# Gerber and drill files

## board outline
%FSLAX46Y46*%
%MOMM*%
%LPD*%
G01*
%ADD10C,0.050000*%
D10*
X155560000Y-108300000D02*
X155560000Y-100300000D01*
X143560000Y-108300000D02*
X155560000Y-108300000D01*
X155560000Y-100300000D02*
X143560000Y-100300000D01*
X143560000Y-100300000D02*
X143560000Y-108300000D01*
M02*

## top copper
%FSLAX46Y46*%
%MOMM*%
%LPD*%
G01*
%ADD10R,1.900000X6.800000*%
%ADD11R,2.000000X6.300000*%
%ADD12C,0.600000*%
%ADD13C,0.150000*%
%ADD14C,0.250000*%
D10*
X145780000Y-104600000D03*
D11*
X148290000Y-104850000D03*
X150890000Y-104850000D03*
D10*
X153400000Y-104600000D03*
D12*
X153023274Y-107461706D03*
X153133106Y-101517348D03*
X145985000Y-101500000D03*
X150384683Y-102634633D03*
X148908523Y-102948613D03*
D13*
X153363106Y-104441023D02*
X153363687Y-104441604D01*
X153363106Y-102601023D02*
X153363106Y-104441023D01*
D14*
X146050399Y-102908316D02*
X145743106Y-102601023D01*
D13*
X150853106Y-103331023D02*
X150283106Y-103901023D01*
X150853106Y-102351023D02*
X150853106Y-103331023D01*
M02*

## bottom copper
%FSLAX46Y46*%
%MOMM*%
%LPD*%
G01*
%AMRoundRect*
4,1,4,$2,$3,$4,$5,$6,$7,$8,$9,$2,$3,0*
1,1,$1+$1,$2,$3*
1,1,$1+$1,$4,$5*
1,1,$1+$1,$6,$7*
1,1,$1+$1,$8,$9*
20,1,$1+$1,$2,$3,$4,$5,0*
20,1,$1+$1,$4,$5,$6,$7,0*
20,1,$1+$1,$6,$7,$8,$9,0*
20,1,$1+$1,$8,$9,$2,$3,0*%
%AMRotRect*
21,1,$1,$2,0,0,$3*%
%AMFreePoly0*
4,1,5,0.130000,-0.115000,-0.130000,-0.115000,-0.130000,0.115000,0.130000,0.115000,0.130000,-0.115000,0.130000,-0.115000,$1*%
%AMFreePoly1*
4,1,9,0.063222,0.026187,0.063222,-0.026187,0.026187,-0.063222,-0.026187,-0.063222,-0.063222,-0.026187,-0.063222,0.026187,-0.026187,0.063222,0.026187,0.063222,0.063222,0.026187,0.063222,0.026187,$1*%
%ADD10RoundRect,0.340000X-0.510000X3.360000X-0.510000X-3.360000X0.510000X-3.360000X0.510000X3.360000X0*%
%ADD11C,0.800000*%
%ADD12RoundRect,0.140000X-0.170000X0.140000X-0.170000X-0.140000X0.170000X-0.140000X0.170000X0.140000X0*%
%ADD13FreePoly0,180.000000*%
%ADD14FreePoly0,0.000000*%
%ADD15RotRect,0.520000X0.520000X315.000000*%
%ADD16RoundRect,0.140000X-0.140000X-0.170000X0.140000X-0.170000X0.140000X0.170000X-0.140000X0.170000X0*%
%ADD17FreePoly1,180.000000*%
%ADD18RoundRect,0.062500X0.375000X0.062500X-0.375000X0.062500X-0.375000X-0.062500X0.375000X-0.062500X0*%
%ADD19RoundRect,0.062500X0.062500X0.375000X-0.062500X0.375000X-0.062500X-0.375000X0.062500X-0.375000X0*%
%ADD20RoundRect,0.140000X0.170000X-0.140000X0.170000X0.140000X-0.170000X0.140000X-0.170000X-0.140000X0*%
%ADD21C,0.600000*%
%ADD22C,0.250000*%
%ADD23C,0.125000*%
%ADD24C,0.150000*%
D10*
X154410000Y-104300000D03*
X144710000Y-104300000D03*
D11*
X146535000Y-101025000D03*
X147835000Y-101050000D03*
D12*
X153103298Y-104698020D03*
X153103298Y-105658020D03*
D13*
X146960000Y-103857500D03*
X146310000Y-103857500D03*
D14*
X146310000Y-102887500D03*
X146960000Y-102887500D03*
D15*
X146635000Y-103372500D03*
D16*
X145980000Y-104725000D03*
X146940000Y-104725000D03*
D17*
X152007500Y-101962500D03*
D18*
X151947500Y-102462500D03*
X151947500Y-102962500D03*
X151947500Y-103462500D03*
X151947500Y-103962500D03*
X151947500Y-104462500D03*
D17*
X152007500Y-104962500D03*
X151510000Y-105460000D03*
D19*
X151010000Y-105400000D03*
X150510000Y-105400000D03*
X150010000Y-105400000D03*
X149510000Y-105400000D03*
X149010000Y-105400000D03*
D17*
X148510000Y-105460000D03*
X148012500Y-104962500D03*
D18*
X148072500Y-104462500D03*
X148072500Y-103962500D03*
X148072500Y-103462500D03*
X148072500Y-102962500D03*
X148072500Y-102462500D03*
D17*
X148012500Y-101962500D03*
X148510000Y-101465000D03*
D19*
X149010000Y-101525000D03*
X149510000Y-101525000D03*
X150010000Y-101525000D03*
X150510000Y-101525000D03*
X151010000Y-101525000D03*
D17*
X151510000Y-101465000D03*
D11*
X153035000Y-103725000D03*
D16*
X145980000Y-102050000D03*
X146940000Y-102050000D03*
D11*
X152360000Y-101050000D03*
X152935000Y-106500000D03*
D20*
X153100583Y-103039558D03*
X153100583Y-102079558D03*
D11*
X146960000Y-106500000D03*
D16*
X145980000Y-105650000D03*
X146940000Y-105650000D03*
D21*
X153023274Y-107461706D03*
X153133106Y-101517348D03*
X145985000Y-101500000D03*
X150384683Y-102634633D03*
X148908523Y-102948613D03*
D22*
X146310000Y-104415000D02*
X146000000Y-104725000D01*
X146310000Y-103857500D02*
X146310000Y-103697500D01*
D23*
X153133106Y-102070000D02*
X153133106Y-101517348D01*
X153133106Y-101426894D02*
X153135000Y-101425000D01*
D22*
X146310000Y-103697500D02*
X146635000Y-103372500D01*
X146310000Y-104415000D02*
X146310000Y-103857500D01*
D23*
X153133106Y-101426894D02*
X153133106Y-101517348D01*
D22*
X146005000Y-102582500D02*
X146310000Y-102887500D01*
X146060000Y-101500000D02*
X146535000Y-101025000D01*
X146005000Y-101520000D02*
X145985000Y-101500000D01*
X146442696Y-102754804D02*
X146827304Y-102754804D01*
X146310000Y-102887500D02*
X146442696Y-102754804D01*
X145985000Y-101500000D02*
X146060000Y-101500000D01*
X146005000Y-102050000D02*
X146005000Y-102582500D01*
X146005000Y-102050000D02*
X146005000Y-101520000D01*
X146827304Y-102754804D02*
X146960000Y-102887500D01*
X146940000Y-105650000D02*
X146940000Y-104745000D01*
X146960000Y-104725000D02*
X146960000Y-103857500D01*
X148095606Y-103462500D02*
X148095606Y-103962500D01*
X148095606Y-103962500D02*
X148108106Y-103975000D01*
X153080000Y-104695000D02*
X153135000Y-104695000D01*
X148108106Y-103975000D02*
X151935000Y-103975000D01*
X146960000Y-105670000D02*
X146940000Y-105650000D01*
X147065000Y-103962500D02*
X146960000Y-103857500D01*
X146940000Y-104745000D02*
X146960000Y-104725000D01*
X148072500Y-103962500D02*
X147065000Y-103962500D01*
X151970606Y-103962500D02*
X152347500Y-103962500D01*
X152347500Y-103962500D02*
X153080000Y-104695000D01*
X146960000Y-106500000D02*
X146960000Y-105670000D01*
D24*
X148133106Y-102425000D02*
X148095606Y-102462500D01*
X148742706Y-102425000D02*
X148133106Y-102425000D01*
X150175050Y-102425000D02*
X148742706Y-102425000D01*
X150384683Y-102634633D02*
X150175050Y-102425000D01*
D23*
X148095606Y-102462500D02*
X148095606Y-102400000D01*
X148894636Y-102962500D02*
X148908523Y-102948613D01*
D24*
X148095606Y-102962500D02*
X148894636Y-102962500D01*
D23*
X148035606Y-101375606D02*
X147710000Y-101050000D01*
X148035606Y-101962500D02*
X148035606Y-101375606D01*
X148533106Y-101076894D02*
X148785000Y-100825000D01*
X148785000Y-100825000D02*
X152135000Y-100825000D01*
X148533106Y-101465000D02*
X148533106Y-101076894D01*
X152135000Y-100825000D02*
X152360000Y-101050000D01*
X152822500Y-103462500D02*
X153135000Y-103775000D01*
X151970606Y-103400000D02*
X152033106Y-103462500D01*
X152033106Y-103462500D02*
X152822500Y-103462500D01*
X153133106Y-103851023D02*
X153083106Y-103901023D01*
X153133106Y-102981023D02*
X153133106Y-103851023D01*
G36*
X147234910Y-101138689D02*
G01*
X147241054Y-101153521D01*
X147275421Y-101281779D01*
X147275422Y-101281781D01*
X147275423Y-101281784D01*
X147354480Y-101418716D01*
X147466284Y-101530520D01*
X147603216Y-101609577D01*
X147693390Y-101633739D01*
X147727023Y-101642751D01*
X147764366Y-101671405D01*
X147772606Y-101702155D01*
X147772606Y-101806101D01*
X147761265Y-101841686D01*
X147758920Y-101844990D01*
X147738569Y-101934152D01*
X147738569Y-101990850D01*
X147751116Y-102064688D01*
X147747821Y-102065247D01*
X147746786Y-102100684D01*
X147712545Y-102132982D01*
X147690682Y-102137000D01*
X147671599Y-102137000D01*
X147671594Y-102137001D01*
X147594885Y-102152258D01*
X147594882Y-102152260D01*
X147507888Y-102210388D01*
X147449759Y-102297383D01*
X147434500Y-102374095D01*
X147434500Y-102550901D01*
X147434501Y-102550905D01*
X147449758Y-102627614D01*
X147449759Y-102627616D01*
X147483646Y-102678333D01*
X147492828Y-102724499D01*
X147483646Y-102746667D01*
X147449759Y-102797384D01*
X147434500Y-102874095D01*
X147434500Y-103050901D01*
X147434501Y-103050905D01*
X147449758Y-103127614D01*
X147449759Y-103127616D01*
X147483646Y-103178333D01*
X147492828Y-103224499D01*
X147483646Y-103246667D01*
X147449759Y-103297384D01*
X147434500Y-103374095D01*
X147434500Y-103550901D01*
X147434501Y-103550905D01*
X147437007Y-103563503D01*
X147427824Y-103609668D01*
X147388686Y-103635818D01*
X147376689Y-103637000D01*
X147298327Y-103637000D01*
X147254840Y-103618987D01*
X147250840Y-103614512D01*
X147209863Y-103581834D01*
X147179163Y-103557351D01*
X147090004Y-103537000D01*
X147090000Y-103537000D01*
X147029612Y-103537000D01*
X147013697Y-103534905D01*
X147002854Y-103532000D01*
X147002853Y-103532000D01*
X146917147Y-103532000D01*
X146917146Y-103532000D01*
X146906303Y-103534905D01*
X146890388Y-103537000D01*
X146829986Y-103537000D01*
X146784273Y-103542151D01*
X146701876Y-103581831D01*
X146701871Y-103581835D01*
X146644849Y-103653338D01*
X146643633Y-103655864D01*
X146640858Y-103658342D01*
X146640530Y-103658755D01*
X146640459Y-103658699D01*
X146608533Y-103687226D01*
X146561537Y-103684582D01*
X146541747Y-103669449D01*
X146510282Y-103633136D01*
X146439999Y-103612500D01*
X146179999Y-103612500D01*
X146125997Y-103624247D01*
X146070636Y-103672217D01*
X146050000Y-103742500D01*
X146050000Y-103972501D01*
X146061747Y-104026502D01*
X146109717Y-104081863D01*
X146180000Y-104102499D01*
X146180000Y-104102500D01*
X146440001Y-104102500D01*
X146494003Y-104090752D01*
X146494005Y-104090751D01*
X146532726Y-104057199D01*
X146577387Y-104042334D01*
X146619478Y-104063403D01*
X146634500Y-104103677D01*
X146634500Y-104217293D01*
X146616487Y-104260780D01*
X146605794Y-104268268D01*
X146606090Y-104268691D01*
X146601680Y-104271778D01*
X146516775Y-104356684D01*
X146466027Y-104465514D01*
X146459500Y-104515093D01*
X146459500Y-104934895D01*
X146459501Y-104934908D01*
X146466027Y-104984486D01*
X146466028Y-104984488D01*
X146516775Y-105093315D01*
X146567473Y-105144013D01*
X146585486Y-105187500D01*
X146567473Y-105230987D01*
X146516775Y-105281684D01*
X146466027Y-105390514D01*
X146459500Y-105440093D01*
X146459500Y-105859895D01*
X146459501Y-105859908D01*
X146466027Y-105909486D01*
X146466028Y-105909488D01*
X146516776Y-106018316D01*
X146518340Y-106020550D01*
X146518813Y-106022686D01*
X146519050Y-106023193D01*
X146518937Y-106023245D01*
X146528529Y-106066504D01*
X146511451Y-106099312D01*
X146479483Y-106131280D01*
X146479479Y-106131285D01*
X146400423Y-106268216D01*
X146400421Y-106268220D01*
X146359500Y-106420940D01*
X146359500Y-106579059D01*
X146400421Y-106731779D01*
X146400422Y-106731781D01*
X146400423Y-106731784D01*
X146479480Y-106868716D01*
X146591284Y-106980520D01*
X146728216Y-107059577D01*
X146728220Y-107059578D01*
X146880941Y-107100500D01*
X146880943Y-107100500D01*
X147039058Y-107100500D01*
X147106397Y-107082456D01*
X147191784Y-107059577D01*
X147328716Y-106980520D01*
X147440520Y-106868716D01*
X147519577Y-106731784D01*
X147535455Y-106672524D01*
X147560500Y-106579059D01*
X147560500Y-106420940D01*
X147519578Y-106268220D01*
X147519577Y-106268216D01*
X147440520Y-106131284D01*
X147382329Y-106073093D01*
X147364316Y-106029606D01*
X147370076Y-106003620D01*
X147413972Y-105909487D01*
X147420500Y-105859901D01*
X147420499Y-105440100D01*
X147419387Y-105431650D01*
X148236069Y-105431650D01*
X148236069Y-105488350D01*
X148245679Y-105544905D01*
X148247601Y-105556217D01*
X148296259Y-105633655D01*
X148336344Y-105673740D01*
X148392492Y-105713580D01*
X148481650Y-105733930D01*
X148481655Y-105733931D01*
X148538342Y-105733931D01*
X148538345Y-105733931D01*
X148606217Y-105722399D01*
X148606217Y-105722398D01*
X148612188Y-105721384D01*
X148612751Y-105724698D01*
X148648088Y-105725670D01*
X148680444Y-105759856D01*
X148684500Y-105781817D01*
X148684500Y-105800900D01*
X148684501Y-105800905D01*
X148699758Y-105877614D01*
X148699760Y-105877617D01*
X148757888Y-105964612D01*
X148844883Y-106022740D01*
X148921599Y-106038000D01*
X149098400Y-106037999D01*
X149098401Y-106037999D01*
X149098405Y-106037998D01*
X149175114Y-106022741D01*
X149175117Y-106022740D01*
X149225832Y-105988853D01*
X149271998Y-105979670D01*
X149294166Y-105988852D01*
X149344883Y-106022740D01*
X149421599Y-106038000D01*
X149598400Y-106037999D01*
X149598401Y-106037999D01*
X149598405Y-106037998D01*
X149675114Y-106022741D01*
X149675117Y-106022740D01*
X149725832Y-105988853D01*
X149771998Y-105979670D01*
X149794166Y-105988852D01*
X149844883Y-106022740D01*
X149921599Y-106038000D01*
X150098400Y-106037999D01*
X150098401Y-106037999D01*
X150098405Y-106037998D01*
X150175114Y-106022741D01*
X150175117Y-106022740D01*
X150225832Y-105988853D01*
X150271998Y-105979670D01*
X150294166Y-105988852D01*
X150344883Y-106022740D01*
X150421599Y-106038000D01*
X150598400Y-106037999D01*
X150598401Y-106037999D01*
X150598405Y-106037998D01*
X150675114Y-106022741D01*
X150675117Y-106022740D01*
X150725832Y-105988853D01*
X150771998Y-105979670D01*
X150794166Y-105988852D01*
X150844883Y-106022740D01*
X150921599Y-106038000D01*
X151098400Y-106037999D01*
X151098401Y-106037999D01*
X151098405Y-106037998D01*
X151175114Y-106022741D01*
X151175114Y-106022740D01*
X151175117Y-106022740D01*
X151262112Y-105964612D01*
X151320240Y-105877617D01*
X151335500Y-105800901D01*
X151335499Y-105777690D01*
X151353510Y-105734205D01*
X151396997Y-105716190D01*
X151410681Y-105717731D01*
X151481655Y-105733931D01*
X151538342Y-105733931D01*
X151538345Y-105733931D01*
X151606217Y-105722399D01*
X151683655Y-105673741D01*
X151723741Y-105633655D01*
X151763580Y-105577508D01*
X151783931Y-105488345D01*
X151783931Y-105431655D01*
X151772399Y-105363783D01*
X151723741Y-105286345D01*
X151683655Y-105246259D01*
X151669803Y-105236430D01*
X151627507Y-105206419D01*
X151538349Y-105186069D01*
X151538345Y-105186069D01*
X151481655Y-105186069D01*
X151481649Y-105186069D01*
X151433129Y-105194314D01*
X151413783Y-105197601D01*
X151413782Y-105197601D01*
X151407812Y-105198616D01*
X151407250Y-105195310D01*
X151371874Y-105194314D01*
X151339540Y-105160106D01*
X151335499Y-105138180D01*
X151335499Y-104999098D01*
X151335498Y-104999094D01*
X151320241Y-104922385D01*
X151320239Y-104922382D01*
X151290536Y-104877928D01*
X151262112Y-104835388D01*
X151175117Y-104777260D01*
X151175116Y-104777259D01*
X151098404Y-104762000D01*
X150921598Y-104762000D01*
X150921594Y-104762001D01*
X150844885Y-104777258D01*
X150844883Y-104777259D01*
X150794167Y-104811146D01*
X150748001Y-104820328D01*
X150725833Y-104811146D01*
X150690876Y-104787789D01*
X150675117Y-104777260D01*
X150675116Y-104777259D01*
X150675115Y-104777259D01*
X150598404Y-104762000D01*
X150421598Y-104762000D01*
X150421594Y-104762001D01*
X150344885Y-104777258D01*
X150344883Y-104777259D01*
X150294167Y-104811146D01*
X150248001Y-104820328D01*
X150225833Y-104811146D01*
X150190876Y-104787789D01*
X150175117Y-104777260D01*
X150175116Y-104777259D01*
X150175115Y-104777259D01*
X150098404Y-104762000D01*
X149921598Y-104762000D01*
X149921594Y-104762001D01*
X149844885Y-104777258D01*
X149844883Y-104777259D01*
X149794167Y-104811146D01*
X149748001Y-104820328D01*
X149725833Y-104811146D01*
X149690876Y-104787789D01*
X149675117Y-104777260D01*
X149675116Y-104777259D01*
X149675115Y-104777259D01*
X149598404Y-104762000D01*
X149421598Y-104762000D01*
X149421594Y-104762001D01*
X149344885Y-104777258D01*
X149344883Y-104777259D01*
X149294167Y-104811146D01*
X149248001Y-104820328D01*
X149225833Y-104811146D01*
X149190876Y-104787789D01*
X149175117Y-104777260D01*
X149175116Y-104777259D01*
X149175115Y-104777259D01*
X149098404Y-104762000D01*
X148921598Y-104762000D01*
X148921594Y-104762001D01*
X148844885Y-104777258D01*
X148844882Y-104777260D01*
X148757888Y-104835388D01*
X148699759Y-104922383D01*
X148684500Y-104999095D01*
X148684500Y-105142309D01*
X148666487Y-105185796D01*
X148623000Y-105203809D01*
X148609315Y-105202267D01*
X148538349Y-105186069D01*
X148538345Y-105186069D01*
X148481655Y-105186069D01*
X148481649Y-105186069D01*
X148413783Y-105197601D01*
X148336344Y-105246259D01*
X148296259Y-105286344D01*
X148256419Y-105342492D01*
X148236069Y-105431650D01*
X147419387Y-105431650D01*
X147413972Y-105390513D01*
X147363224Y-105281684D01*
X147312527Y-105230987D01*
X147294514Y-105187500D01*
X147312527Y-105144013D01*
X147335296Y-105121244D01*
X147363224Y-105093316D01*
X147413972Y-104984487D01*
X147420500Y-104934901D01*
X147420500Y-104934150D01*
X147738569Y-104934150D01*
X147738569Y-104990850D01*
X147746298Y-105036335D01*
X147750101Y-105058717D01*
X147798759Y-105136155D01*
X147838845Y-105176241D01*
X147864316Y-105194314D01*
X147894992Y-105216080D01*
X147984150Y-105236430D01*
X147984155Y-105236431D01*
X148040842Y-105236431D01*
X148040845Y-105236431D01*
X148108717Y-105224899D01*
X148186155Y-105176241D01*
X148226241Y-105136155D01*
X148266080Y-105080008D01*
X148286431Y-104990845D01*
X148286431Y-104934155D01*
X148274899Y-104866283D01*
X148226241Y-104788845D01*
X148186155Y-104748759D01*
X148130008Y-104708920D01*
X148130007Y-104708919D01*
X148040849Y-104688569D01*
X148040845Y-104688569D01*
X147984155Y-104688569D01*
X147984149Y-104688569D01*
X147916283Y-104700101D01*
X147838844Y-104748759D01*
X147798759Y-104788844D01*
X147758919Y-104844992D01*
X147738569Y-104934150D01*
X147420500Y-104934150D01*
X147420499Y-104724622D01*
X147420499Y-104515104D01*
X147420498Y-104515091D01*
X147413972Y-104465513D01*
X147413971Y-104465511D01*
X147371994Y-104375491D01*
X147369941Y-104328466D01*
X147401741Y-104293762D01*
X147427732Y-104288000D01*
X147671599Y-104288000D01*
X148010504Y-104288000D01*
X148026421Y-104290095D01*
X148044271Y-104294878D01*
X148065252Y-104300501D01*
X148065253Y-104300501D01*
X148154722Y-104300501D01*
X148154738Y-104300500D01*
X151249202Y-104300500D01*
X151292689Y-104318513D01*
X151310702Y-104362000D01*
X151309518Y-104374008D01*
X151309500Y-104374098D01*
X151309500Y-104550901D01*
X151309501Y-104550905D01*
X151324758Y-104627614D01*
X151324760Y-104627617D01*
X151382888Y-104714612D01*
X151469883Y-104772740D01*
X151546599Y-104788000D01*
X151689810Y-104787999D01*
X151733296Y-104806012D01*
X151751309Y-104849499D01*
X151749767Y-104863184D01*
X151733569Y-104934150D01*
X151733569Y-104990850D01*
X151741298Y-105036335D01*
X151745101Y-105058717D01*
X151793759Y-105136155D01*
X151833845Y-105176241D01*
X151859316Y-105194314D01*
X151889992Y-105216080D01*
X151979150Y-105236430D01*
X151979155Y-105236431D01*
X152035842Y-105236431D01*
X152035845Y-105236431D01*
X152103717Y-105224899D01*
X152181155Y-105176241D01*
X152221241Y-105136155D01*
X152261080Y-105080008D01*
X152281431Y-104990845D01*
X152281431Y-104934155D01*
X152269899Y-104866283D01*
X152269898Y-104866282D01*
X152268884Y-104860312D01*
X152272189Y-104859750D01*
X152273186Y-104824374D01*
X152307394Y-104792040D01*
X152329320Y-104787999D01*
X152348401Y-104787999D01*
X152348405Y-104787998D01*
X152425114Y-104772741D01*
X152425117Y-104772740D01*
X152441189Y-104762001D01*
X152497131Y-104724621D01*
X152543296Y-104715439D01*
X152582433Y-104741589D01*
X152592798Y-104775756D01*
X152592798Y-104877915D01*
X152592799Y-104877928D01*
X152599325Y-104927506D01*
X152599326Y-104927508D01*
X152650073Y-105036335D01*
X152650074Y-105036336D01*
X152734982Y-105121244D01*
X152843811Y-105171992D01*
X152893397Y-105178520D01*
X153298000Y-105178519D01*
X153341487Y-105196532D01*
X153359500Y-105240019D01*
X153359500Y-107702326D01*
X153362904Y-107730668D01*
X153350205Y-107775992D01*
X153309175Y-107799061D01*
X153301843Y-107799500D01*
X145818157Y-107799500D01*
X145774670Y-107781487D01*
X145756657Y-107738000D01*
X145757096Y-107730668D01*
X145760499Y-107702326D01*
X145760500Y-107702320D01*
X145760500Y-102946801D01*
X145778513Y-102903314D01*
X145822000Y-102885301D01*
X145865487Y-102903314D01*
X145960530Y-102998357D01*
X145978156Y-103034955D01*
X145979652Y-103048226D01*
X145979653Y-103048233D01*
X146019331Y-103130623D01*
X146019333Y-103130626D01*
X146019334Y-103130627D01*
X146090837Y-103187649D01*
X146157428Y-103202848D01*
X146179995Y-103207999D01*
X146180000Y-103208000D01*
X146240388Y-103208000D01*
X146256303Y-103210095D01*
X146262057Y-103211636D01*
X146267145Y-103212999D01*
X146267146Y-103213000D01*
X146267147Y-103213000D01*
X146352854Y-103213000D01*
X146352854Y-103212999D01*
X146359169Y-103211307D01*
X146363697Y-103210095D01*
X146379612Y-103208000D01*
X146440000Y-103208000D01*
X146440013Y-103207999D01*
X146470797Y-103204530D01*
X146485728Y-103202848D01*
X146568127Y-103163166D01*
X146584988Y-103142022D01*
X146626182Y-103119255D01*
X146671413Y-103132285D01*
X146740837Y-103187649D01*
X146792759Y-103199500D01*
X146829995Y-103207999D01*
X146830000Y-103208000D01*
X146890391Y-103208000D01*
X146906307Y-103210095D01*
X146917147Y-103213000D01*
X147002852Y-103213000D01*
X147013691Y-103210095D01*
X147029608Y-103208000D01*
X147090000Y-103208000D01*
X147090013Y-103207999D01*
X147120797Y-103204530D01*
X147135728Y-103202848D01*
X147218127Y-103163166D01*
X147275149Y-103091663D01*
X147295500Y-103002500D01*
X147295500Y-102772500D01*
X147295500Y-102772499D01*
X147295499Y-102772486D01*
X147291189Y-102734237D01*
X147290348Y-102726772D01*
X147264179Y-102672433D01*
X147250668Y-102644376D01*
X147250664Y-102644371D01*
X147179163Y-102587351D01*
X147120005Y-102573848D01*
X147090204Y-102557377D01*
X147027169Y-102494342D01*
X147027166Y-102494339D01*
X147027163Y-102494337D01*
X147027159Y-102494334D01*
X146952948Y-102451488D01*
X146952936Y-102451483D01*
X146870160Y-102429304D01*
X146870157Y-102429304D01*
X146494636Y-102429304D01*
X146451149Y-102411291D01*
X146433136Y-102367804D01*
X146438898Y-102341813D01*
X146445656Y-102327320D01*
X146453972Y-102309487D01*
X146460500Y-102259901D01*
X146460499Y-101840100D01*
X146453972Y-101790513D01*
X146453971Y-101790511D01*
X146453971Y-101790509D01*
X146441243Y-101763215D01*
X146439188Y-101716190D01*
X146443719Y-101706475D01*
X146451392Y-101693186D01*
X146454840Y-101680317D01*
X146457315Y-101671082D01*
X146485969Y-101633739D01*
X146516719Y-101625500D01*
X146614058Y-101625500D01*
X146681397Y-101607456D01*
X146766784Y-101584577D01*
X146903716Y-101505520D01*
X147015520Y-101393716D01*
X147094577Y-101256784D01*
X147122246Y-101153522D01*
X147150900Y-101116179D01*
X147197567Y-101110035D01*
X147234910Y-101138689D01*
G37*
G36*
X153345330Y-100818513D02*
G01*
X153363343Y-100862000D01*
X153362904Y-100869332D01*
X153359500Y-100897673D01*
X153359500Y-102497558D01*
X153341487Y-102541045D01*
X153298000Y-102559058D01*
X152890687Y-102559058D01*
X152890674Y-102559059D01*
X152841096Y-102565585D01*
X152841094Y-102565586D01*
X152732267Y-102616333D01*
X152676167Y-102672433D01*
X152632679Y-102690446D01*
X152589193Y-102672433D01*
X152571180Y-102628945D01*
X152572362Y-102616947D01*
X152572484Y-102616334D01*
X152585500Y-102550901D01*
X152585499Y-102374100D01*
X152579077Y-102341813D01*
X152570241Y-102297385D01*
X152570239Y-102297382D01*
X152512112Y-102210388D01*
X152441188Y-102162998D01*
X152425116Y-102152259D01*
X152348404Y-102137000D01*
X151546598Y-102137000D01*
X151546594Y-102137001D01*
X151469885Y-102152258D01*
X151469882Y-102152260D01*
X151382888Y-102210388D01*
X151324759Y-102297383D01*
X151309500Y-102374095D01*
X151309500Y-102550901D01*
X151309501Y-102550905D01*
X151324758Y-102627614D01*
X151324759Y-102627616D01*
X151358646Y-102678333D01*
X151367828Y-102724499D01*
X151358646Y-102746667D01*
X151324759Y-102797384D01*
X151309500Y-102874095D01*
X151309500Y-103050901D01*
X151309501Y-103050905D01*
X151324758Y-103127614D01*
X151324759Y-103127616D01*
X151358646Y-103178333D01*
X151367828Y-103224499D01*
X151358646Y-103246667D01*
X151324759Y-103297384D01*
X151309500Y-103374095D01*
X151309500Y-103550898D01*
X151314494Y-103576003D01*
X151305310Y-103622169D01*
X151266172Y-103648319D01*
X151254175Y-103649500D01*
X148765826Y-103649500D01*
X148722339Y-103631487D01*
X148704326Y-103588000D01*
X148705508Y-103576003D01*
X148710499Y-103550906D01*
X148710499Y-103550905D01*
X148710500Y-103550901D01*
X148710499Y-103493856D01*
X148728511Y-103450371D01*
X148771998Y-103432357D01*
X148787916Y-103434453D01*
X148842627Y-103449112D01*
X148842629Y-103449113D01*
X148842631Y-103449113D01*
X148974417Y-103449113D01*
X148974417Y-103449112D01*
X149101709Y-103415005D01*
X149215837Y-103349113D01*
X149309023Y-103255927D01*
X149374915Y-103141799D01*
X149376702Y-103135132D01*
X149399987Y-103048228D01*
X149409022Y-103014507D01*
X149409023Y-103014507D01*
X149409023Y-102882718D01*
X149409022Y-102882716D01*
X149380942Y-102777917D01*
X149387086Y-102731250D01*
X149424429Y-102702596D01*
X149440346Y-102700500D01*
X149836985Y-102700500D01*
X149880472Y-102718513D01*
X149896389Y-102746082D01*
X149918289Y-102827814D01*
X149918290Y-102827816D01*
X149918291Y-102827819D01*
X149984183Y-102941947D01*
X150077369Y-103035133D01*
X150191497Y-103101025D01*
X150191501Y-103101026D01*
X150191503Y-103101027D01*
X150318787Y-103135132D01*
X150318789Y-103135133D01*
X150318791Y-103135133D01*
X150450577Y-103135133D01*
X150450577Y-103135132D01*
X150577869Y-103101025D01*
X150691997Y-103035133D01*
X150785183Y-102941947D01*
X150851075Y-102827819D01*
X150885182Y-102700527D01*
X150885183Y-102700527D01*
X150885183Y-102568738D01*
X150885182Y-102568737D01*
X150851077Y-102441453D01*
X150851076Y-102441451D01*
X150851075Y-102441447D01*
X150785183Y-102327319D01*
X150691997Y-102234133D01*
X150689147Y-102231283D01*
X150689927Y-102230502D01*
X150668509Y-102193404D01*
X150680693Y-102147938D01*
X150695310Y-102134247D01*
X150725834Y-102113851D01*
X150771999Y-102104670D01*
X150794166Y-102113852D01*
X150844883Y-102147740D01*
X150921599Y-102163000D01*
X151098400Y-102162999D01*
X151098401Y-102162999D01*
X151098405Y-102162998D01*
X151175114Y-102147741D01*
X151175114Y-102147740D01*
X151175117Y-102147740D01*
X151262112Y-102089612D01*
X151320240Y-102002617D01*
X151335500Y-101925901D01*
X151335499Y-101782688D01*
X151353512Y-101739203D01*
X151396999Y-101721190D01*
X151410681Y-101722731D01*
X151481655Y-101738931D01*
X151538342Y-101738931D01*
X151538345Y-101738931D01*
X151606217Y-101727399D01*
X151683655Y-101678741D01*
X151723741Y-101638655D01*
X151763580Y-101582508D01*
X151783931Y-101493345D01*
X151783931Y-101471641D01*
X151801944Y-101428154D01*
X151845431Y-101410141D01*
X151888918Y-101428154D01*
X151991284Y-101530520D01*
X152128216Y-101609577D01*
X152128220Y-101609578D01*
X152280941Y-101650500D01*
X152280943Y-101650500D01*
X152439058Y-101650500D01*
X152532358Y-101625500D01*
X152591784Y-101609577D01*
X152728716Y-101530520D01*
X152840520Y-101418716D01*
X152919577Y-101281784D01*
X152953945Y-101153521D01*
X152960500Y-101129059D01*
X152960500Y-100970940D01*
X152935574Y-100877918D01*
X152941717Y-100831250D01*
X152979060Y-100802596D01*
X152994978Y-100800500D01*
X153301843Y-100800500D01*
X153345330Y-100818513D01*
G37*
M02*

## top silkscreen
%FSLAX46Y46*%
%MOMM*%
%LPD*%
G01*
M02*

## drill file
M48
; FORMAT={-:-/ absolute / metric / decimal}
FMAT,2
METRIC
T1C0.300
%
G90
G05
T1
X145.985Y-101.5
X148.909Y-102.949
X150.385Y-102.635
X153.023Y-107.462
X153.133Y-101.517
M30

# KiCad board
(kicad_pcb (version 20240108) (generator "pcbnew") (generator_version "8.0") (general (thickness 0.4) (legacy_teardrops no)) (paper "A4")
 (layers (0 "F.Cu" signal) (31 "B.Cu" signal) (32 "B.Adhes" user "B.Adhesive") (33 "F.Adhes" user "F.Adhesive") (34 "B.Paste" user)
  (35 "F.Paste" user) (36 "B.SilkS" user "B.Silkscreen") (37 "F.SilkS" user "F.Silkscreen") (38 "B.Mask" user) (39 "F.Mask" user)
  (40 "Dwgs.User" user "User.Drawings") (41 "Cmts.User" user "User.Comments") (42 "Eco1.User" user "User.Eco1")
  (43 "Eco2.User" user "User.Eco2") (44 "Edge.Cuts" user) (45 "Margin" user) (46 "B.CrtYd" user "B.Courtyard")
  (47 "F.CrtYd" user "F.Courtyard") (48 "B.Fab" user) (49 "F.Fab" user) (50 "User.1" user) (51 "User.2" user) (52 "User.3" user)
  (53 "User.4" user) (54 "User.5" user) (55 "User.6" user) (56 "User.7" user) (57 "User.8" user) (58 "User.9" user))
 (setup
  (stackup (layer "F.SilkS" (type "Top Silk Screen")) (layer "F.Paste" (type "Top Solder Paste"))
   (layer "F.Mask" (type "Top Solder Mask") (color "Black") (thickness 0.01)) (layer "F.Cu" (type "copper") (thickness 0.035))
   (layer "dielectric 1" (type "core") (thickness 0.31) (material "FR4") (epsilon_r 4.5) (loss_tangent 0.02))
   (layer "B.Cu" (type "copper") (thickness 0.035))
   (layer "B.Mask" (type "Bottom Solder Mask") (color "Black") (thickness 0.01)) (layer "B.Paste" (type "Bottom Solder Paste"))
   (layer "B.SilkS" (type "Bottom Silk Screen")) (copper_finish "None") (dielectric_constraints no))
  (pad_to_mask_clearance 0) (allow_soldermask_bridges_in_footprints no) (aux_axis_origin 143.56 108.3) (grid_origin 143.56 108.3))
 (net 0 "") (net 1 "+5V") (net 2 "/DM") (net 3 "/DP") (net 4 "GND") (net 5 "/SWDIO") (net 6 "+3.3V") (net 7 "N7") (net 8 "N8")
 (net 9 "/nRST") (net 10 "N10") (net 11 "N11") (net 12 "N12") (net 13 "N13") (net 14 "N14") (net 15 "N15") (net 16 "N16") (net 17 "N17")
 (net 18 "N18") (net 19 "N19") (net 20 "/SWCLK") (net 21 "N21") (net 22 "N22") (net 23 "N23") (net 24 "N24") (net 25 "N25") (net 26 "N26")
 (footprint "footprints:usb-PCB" (layer "F.Cu") (at 149.59 100.3 180)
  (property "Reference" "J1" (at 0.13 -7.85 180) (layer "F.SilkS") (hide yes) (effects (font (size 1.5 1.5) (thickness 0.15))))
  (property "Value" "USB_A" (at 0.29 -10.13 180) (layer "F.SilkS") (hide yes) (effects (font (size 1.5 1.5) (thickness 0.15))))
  (pad "1" connect rect (at 3.81 -4.3 180) (size 1.9 6.8) (layers "F.Cu" "F.Mask") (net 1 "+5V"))
  (pad "2" connect rect (at 1.3 -4.55 180) (size 2 6.3) (layers "F.Cu" "F.Mask") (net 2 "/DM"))
  (pad "3" connect rect (at -1.3 -4.55 180) (size 2 6.3) (layers "F.Cu" "F.Mask") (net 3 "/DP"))
  (pad "4" connect rect (at -3.81 -4.3 180) (size 1.9 6.8) (layers "F.Cu" "F.Mask") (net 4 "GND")))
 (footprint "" (layer "F.Cu") (at 154.552655 104.23372)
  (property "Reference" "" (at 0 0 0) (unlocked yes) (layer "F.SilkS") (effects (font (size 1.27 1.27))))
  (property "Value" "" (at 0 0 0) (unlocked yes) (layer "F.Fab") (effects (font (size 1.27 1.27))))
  (pad "1" smd roundrect (at -0.142655 0.06628 270) (size 7.4 1.7) (layers "B.Cu" "B.Mask") (roundrect_rratio 0.2)))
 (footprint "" (layer "F.Cu") (at 144.66 104.23)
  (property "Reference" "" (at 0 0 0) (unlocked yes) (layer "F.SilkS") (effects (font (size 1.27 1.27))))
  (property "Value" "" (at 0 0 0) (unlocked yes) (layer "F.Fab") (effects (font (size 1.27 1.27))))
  (pad "1" smd roundrect (at 0.05 0.07 270) (size 7.4 1.7) (layers "B.Cu" "B.Mask") (roundrect_rratio 0.2)))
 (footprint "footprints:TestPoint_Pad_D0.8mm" (layer "B.Cu") (at 146.535 101.025 180)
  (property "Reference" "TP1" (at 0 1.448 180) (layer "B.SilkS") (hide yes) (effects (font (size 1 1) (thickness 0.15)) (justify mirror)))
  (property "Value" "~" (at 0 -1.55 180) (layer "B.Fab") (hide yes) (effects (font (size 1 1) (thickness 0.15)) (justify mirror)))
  (pad "1" smd circle (at 0 0 180) (size 0.8 0.8) (layers "B.Cu" "B.Mask") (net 1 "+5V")))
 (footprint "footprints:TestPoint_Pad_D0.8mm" (layer "B.Cu") (at 147.835 102.436009)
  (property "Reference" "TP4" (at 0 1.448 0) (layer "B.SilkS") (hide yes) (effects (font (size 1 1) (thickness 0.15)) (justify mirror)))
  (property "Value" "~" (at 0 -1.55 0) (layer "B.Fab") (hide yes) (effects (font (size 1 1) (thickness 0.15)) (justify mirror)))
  (pad "1" smd circle (at 0 -1.386009) (size 0.8 0.8) (layers "B.Cu" "B.Mask") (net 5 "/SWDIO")))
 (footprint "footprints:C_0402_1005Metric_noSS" (layer "B.Cu") (at 153.103298 105.17802 -90)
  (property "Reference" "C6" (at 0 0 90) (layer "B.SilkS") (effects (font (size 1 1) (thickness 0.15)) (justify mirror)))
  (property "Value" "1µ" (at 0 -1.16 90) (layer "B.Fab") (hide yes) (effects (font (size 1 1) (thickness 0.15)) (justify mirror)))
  (pad "1" smd roundrect (at -0.48 0 270) (size 0.56 0.62) (layers "B.Cu" "B.Paste" "B.Mask") (roundrect_rratio 0.25) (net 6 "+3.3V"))
  (pad "2" smd roundrect (at 0.48 0 270) (size 0.56 0.62) (layers "B.Cu" "B.Paste" "B.Mask") (roundrect_rratio 0.25) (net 4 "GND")))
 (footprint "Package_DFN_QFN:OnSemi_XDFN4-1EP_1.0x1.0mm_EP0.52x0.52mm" (layer "B.Cu") (at 146.635 103.3725 90)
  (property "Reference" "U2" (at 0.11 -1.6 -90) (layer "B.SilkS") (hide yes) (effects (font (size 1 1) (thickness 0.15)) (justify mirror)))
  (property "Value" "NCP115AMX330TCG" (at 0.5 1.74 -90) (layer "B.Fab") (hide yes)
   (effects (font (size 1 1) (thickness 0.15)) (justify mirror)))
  (pad "1" smd custom (at -0.485 0.325 180) (size 0.26 0.23) (layers "B.Cu" "B.Paste" "B.Mask") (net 6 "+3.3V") (zone_connect 0)
   (thermal_bridge_angle 45) (options (clearance outline) (anchor rect)) (primitives))
  (pad "2" smd custom (at -0.485 -0.325 180) (size 0.26 0.23) (layers "B.Cu" "B.Paste" "B.Mask") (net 4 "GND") (zone_connect 0)
   (thermal_bridge_angle 45) (options (clearance outline) (anchor rect)) (primitives))
  (pad "3" smd custom (at 0.485 -0.325) (size 0.26 0.23) (layers "B.Cu" "B.Paste" "B.Mask") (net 1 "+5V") (zone_connect 0)
   (thermal_bridge_angle 45) (options (clearance outline) (anchor rect)) (primitives))
  (pad "4" smd custom (at 0.485 0.325) (size 0.26 0.23) (layers "B.Cu" "B.Paste" "B.Mask") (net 1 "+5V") (zone_connect 0)
   (thermal_bridge_angle 45) (options (clearance outline) (anchor rect)) (primitives))
  (pad "5" smd rect (at 0 0 315) (size 0.52 0.52) (layers "B.Cu" "B.Paste" "B.Mask") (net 4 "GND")))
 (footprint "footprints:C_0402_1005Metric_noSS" (layer "B.Cu") (at 146.46 104.725)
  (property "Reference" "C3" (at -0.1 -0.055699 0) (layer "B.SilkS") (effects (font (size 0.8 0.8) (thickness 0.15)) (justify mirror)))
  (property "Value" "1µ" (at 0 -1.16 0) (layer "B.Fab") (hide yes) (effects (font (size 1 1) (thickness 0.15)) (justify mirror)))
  (pad "1" smd roundrect (at -0.48 0) (size 0.56 0.62) (layers "B.Cu" "B.Paste" "B.Mask") (roundrect_rratio 0.25) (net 4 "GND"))
  (pad "2" smd roundrect (at 0.48 0) (size 0.56 0.62) (layers "B.Cu" "B.Paste" "B.Mask") (roundrect_rratio 0.25) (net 6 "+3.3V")))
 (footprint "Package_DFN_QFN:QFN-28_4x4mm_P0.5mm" (layer "B.Cu") (at 150.01 103.4625 180)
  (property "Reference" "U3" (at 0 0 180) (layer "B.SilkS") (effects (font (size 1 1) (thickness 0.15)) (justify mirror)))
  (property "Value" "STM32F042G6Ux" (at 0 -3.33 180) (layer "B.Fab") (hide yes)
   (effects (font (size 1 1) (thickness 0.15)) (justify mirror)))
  (pad "1" smd custom (at -1.9975 1.5 180) (size 0.136863 0.136863) (layers "B.Cu" "B.Paste" "B.Mask") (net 4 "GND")
   (options (clearance outline) (anchor circle)) (primitives))
  (pad "2" smd roundrect (at -1.9375 1 180) (size 0.875 0.25) (layers "B.Cu" "B.Paste" "B.Mask") (roundrect_rratio 0.25) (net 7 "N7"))
  (pad "3" smd roundrect (at -1.9375 0.5 180) (size 0.875 0.25) (layers "B.Cu" "B.Paste" "B.Mask") (roundrect_rratio 0.25) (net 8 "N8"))
  (pad "4" smd roundrect (at -1.9375 0 180) (size 0.875 0.25) (layers "B.Cu" "B.Paste" "B.Mask") (roundrect_rratio 0.25) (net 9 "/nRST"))
  (pad "5" smd roundrect (at -1.9375 -0.5 180) (size 0.875 0.25) (layers "B.Cu" "B.Paste" "B.Mask") (roundrect_rratio 0.25) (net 6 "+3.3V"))
  (pad "6" smd roundrect (at -1.9375 -1 180) (size 0.875 0.25) (layers "B.Cu" "B.Paste" "B.Mask") (roundrect_rratio 0.25) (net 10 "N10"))
  (pad "7" smd custom (at -1.9975 -1.5 180) (size 0.136863 0.136863) (layers "B.Cu" "B.Paste" "B.Mask") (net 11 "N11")
   (options (clearance outline) (anchor circle)) (primitives))
  (pad "8" smd custom (at -1.5 -1.9975 180) (size 0.136863 0.136863) (layers "B.Cu" "B.Paste" "B.Mask") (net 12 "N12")
   (options (clearance outline) (anchor circle)) (primitives))
  (pad "9" smd roundrect (at -1 -1.9375 180) (size 0.25 0.875) (layers "B.Cu" "B.Paste" "B.Mask") (roundrect_rratio 0.25) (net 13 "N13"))
  (pad "10" smd roundrect (at -0.5 -1.9375 180) (size 0.25 0.875) (layers "B.Cu" "B.Paste" "B.Mask") (roundrect_rratio 0.25) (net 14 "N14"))
  (pad "11" smd roundrect (at 0 -1.9375 180) (size 0.25 0.875) (layers "B.Cu" "B.Paste" "B.Mask") (roundrect_rratio 0.25) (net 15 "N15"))
  (pad "12" smd roundrect (at 0.5 -1.9375 180) (size 0.25 0.875) (layers "B.Cu" "B.Paste" "B.Mask") (roundrect_rratio 0.25) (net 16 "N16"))
  (pad "13" smd roundrect (at 1 -1.9375 180) (size 0.25 0.875) (layers "B.Cu" "B.Paste" "B.Mask") (roundrect_rratio 0.25) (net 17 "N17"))
  (pad "14" smd custom (at 1.5 -1.9975 180) (size 0.136863 0.136863) (layers "B.Cu" "B.Paste" "B.Mask") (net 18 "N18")
   (options (clearance outline) (anchor circle)) (primitives))
  (pad "15" smd custom (at 1.9975 -1.5 180) (size 0.136863 0.136863) (layers "B.Cu" "B.Paste" "B.Mask") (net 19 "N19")
   (options (clearance outline) (anchor circle)) (primitives))
  (pad "16" smd roundrect (at 1.9375 -1 180) (size 0.875 0.25) (layers "B.Cu" "B.Paste" "B.Mask") (roundrect_rratio 0.25) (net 4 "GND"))
  (pad "17" smd roundrect (at 1.9375 -0.5 180) (size 0.875 0.25) (layers "B.Cu" "B.Paste" "B.Mask") (roundrect_rratio 0.25) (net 6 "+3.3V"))
  (pad "18" smd roundrect (at 1.9375 0 180) (size 0.875 0.25) (layers "B.Cu" "B.Paste" "B.Mask") (roundrect_rratio 0.25) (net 6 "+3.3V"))
  (pad "19" smd roundrect (at 1.9375 0.5 180) (size 0.875 0.25) (layers "B.Cu" "B.Paste" "B.Mask") (roundrect_rratio 0.25) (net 2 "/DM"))
  (pad "20" smd roundrect (at 1.9375 1 180) (size 0.875 0.25) (layers "B.Cu" "B.Paste" "B.Mask") (roundrect_rratio 0.25) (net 3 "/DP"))
  (pad "21" smd custom (at 1.9975 1.5 180) (size 0.136863 0.136863) (layers "B.Cu" "B.Paste" "B.Mask") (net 5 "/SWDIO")
   (options (clearance outline) (anchor circle)) (primitives))
  (pad "22" smd custom (at 1.5 1.9975 180) (size 0.136863 0.136863) (layers "B.Cu" "B.Paste" "B.Mask") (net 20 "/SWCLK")
   (options (clearance outline) (anchor circle)) (primitives))
  (pad "23" smd roundrect (at 1 1.9375 180) (size 0.25 0.875) (layers "B.Cu" "B.Paste" "B.Mask") (roundrect_rratio 0.25) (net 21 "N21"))
  (pad "24" smd roundrect (at 0.5 1.9375 180) (size 0.25 0.875) (layers "B.Cu" "B.Paste" "B.Mask") (roundrect_rratio 0.25) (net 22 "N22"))
  (pad "25" smd roundrect (at 0 1.9375 180) (size 0.25 0.875) (layers "B.Cu" "B.Paste" "B.Mask") (roundrect_rratio 0.25) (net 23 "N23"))
  (pad "26" smd roundrect (at -0.5 1.9375 180) (size 0.25 0.875) (layers "B.Cu" "B.Paste" "B.Mask") (roundrect_rratio 0.25) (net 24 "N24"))
  (pad "27" smd roundrect (at -1 1.9375 180) (size 0.25 0.875) (layers "B.Cu" "B.Paste" "B.Mask") (roundrect_rratio 0.25) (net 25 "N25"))
  (pad "28" smd custom (at -1.5 1.9975 180) (size 0.136863 0.136863) (layers "B.Cu" "B.Paste" "B.Mask") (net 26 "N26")
   (options (clearance outline) (anchor circle)) (primitives)))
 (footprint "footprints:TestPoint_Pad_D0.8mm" (layer "B.Cu") (at 152.835 103.725)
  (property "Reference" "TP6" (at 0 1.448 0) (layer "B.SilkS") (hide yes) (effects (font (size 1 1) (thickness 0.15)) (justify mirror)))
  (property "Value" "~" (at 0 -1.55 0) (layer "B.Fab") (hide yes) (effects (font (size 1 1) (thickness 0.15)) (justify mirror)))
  (pad "1" smd circle (at 0.2 0) (size 0.8 0.8) (layers "B.Cu" "B.Mask") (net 9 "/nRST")))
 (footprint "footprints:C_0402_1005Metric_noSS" (layer "B.Cu") (at 146.46 102.05)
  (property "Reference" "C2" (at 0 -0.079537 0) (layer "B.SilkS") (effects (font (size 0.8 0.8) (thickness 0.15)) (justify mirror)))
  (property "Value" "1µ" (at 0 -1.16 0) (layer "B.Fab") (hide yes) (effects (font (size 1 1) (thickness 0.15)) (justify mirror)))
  (pad "1" smd roundrect (at -0.48 0) (size 0.56 0.62) (layers "B.Cu" "B.Paste" "B.Mask") (roundrect_rratio 0.25) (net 1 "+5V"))
  (pad "2" smd roundrect (at 0.48 0) (size 0.56 0.62) (layers "B.Cu" "B.Paste" "B.Mask") (roundrect_rratio 0.25) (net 4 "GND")))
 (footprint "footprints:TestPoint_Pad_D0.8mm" (layer "B.Cu") (at 152.36 100.87487)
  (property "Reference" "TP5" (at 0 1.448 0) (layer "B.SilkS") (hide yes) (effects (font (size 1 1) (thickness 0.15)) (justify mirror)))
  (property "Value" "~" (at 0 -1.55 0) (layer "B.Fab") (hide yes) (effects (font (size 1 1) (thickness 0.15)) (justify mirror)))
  (pad "1" smd circle (at 0 0.17513) (size 0.8 0.8) (layers "B.Cu" "B.Mask") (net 20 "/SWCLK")))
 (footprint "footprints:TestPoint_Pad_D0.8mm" (layer "B.Cu") (at 152.935 106.325 180)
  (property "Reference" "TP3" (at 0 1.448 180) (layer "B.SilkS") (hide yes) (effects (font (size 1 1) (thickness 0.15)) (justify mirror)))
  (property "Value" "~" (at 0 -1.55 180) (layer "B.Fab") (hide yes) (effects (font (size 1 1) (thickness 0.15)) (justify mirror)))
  (pad "1" smd circle (at 0 -0.175 180) (size 0.8 0.8) (layers "B.Cu" "B.Mask") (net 4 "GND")))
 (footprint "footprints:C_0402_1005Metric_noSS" (layer "B.Cu") (at 153.100583 102.559558 90)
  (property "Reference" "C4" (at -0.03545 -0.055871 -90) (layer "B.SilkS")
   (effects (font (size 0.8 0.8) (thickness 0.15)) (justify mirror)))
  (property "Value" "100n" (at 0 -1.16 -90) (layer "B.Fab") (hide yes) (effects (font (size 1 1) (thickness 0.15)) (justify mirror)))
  (pad "1" smd roundrect (at -0.48 0 90) (size 0.56 0.62) (layers "B.Cu" "B.Paste" "B.Mask") (roundrect_rratio 0.25) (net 9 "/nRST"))
  (pad "2" smd roundrect (at 0.48 0 90) (size 0.56 0.62) (layers "B.Cu" "B.Paste" "B.Mask") (roundrect_rratio 0.25) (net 4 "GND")))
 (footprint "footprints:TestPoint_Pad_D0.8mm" (layer "B.Cu") (at 146.96 106.5)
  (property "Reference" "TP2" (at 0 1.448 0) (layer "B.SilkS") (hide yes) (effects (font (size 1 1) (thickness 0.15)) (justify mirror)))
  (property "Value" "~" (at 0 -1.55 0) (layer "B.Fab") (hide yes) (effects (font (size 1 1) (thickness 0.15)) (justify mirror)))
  (pad "1" smd circle (at 0 0) (size 0.8 0.8) (layers "B.Cu" "B.Mask") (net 6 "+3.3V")))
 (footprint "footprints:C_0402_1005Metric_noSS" (layer "B.Cu") (at 146.46 105.65)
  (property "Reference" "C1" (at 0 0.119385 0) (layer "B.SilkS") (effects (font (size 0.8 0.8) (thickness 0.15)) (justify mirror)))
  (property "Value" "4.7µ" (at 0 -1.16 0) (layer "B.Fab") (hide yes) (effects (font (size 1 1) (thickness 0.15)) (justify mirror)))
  (pad "1" smd roundrect (at -0.48 0) (size 0.56 0.62) (layers "B.Cu" "B.Paste" "B.Mask") (roundrect_rratio 0.25) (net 4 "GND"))
  (pad "2" smd roundrect (at 0.48 0) (size 0.56 0.62) (layers "B.Cu" "B.Paste" "B.Mask") (roundrect_rratio 0.25) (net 6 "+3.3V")))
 (gr_line (start 155.56 108.3) (end 155.56 100.3) (stroke (width 0.05) (type default)) (layer "Edge.Cuts"))
 (gr_line (start 143.56 108.3) (end 155.56 108.3) (stroke (width 0.05) (type default)) (layer "Edge.Cuts"))
 (gr_line (start 155.56 100.3) (end 143.56 100.3) (stroke (width 0.05) (type default)) (layer "Edge.Cuts"))
 (gr_line (start 143.56 100.3) (end 143.56 108.3) (stroke (width 0.05) (type default)) (layer "Edge.Cuts"))
 (segment (start 153.363106 104.441023) (end 153.363687 104.441604) (width 0.15) (layer "F.Cu") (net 4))
 (segment (start 153.363106 102.601023) (end 153.363106 104.441023) (width 0.15) (layer "F.Cu") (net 4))
 (via (at 153.023274 107.461706) (size 0.6) (drill 0.3) (layers "F.Cu" "B.Cu") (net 4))
 (via (at 153.133106 101.517348) (size 0.6) (drill 0.3) (layers "F.Cu" "B.Cu") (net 4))
 (segment (start 146.31 104.415) (end 146 104.725) (width 0.25) (layer "B.Cu") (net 4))
 (segment (start 146.31 103.8575) (end 146.31 103.6975) (width 0.25) (layer "B.Cu") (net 4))
 (segment (start 153.133106 102.07) (end 153.133106 101.517348) (width 0.125) (layer "B.Cu") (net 4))
 (segment (start 153.133106 101.426894) (end 153.135 101.425) (width 0.125) (layer "B.Cu") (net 4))
 (segment (start 146.31 103.6975) (end 146.635 103.3725) (width 0.25) (layer "B.Cu") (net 4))
 (segment (start 146.31 104.415) (end 146.31 103.8575) (width 0.25) (layer "B.Cu") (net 4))
 (segment (start 153.133106 101.426894) (end 153.133106 101.517348) (width 0.125) (layer "B.Cu") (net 4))
 (segment (start 146.050399 102.908316) (end 145.743106 102.601023) (width 0.25) (layer "F.Cu") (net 1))
 (via (at 145.985 101.5) (size 0.6) (drill 0.3) (layers "F.Cu" "B.Cu") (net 1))
 (segment (start 146.005 102.5825) (end 146.31 102.8875) (width 0.25) (layer "B.Cu") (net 1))
 (segment (start 146.06 101.5) (end 146.535 101.025) (width 0.25) (layer "B.Cu") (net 1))
 (segment (start 146.005 101.52) (end 145.985 101.5) (width 0.25) (layer "B.Cu") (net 1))
 (segment (start 146.442696 102.754804) (end 146.827304 102.754804) (width 0.25) (layer "B.Cu") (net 1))
 (segment (start 146.31 102.8875) (end 146.442696 102.754804) (width 0.25) (layer "B.Cu") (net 1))
 (segment (start 145.985 101.5) (end 146.06 101.5) (width 0.25) (layer "B.Cu") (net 1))
 (segment (start 146.005 102.05) (end 146.005 102.5825) (width 0.25) (layer "B.Cu") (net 1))
 (segment (start 146.005 102.05) (end 146.005 101.52) (width 0.25) (layer "B.Cu") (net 1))
 (segment (start 146.827304 102.754804) (end 146.96 102.8875) (width 0.25) (layer "B.Cu") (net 1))
 (segment (start 146.94 105.65) (end 146.94 104.745) (width 0.25) (layer "B.Cu") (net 6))
 (segment (start 146.96 104.725) (end 146.96 103.8575) (width 0.25) (layer "B.Cu") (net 6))
 (segment (start 148.095606 103.4625) (end 148.095606 103.9625) (width 0.25) (layer "B.Cu") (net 6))
 (segment (start 148.095606 103.9625) (end 148.108106 103.975) (width 0.25) (layer "B.Cu") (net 6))
 (segment (start 153.08 104.695) (end 153.135 104.695) (width 0.25) (layer "B.Cu") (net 6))
 (segment (start 148.108106 103.975) (end 151.935 103.975) (width 0.25) (layer "B.Cu") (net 6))
 (segment (start 146.96 105.67) (end 146.94 105.65) (width 0.25) (layer "B.Cu") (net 6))
 (segment (start 147.065 103.9625) (end 146.96 103.8575) (width 0.25) (layer "B.Cu") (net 6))
 (segment (start 146.94 104.745) (end 146.96 104.725) (width 0.25) (layer "B.Cu") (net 6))
 (segment (start 148.0725 103.9625) (end 147.065 103.9625) (width 0.25) (layer "B.Cu") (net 6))
 (segment (start 151.970606 103.9625) (end 152.3475 103.9625) (width 0.25) (layer "B.Cu") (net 6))
 (segment (start 152.3475 103.9625) (end 153.08 104.695) (width 0.25) (layer "B.Cu") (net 6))
 (segment (start 146.96 106.5) (end 146.96 105.67) (width 0.25) (layer "B.Cu") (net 6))
 (segment (start 150.853106 103.331023) (end 150.283106 103.901023) (width 0.15) (layer "F.Cu") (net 3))
 (segment (start 150.853106 102.351023) (end 150.853106 103.331023) (width 0.15) (layer "F.Cu") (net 3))
 (via (at 150.384683 102.634633) (size 0.6) (drill 0.3) (layers "F.Cu" "B.Cu") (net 3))
 (segment (start 148.133106 102.425) (end 148.095606 102.4625) (width 0.15) (layer "B.Cu") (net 3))
 (segment (start 148.742706 102.425) (end 148.133106 102.425) (width 0.15) (layer "B.Cu") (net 3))
 (segment (start 150.17505 102.425) (end 148.742706 102.425) (width 0.15) (layer "B.Cu") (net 3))
 (segment (start 150.384683 102.634633) (end 150.17505 102.425) (width 0.15) (layer "B.Cu") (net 3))
 (segment (start 148.095606 102.4625) (end 148.095606 102.4) (width 0.125) (layer "B.Cu") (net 3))
 (via (at 148.908523 102.948613) (size 0.6) (drill 0.3) (layers "F.Cu" "B.Cu") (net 2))
 (segment (start 148.894636 102.9625) (end 148.908523 102.948613) (width 0.125) (layer "B.Cu") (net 2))
 (segment (start 148.095606 102.9625) (end 148.894636 102.9625) (width 0.15) (layer "B.Cu") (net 2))
 (segment (start 148.035606 101.375606) (end 147.71 101.05) (width 0.125) (layer "B.Cu") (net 5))
 (segment (start 148.035606 101.9625) (end 148.035606 101.375606) (width 0.125) (layer "B.Cu") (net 5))
 (segment (start 148.533106 101.076894) (end 148.785 100.825) (width 0.125) (layer "B.Cu") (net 20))
 (segment (start 148.785 100.825) (end 152.135 100.825) (width 0.125) (layer "B.Cu") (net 20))
 (segment (start 148.533106 101.465) (end 148.533106 101.076894) (width 0.125) (layer "B.Cu") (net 20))
 (segment (start 152.135 100.825) (end 152.36 101.05) (width 0.125) (layer "B.Cu") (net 20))
 (segment (start 152.8225 103.4625) (end 153.135 103.775) (width 0.125) (layer "B.Cu") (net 9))
 (segment (start 151.970606 103.4) (end 152.033106 103.4625) (width 0.125) (layer "B.Cu") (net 9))
 (segment (start 152.033106 103.4625) (end 152.8225 103.4625) (width 0.125) (layer "B.Cu") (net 9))
 (segment (start 153.133106 103.851023) (end 153.083106 103.901023) (width 0.125) (layer "B.Cu") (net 9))
 (segment (start 153.133106 102.981023) (end 153.133106 103.851023) (width 0.125) (layer "B.Cu") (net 9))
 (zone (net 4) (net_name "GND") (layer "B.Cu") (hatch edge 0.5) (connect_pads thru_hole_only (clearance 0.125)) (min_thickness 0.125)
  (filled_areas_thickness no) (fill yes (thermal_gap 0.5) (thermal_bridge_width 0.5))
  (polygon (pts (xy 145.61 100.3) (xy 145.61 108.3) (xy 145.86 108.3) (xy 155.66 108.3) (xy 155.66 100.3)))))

